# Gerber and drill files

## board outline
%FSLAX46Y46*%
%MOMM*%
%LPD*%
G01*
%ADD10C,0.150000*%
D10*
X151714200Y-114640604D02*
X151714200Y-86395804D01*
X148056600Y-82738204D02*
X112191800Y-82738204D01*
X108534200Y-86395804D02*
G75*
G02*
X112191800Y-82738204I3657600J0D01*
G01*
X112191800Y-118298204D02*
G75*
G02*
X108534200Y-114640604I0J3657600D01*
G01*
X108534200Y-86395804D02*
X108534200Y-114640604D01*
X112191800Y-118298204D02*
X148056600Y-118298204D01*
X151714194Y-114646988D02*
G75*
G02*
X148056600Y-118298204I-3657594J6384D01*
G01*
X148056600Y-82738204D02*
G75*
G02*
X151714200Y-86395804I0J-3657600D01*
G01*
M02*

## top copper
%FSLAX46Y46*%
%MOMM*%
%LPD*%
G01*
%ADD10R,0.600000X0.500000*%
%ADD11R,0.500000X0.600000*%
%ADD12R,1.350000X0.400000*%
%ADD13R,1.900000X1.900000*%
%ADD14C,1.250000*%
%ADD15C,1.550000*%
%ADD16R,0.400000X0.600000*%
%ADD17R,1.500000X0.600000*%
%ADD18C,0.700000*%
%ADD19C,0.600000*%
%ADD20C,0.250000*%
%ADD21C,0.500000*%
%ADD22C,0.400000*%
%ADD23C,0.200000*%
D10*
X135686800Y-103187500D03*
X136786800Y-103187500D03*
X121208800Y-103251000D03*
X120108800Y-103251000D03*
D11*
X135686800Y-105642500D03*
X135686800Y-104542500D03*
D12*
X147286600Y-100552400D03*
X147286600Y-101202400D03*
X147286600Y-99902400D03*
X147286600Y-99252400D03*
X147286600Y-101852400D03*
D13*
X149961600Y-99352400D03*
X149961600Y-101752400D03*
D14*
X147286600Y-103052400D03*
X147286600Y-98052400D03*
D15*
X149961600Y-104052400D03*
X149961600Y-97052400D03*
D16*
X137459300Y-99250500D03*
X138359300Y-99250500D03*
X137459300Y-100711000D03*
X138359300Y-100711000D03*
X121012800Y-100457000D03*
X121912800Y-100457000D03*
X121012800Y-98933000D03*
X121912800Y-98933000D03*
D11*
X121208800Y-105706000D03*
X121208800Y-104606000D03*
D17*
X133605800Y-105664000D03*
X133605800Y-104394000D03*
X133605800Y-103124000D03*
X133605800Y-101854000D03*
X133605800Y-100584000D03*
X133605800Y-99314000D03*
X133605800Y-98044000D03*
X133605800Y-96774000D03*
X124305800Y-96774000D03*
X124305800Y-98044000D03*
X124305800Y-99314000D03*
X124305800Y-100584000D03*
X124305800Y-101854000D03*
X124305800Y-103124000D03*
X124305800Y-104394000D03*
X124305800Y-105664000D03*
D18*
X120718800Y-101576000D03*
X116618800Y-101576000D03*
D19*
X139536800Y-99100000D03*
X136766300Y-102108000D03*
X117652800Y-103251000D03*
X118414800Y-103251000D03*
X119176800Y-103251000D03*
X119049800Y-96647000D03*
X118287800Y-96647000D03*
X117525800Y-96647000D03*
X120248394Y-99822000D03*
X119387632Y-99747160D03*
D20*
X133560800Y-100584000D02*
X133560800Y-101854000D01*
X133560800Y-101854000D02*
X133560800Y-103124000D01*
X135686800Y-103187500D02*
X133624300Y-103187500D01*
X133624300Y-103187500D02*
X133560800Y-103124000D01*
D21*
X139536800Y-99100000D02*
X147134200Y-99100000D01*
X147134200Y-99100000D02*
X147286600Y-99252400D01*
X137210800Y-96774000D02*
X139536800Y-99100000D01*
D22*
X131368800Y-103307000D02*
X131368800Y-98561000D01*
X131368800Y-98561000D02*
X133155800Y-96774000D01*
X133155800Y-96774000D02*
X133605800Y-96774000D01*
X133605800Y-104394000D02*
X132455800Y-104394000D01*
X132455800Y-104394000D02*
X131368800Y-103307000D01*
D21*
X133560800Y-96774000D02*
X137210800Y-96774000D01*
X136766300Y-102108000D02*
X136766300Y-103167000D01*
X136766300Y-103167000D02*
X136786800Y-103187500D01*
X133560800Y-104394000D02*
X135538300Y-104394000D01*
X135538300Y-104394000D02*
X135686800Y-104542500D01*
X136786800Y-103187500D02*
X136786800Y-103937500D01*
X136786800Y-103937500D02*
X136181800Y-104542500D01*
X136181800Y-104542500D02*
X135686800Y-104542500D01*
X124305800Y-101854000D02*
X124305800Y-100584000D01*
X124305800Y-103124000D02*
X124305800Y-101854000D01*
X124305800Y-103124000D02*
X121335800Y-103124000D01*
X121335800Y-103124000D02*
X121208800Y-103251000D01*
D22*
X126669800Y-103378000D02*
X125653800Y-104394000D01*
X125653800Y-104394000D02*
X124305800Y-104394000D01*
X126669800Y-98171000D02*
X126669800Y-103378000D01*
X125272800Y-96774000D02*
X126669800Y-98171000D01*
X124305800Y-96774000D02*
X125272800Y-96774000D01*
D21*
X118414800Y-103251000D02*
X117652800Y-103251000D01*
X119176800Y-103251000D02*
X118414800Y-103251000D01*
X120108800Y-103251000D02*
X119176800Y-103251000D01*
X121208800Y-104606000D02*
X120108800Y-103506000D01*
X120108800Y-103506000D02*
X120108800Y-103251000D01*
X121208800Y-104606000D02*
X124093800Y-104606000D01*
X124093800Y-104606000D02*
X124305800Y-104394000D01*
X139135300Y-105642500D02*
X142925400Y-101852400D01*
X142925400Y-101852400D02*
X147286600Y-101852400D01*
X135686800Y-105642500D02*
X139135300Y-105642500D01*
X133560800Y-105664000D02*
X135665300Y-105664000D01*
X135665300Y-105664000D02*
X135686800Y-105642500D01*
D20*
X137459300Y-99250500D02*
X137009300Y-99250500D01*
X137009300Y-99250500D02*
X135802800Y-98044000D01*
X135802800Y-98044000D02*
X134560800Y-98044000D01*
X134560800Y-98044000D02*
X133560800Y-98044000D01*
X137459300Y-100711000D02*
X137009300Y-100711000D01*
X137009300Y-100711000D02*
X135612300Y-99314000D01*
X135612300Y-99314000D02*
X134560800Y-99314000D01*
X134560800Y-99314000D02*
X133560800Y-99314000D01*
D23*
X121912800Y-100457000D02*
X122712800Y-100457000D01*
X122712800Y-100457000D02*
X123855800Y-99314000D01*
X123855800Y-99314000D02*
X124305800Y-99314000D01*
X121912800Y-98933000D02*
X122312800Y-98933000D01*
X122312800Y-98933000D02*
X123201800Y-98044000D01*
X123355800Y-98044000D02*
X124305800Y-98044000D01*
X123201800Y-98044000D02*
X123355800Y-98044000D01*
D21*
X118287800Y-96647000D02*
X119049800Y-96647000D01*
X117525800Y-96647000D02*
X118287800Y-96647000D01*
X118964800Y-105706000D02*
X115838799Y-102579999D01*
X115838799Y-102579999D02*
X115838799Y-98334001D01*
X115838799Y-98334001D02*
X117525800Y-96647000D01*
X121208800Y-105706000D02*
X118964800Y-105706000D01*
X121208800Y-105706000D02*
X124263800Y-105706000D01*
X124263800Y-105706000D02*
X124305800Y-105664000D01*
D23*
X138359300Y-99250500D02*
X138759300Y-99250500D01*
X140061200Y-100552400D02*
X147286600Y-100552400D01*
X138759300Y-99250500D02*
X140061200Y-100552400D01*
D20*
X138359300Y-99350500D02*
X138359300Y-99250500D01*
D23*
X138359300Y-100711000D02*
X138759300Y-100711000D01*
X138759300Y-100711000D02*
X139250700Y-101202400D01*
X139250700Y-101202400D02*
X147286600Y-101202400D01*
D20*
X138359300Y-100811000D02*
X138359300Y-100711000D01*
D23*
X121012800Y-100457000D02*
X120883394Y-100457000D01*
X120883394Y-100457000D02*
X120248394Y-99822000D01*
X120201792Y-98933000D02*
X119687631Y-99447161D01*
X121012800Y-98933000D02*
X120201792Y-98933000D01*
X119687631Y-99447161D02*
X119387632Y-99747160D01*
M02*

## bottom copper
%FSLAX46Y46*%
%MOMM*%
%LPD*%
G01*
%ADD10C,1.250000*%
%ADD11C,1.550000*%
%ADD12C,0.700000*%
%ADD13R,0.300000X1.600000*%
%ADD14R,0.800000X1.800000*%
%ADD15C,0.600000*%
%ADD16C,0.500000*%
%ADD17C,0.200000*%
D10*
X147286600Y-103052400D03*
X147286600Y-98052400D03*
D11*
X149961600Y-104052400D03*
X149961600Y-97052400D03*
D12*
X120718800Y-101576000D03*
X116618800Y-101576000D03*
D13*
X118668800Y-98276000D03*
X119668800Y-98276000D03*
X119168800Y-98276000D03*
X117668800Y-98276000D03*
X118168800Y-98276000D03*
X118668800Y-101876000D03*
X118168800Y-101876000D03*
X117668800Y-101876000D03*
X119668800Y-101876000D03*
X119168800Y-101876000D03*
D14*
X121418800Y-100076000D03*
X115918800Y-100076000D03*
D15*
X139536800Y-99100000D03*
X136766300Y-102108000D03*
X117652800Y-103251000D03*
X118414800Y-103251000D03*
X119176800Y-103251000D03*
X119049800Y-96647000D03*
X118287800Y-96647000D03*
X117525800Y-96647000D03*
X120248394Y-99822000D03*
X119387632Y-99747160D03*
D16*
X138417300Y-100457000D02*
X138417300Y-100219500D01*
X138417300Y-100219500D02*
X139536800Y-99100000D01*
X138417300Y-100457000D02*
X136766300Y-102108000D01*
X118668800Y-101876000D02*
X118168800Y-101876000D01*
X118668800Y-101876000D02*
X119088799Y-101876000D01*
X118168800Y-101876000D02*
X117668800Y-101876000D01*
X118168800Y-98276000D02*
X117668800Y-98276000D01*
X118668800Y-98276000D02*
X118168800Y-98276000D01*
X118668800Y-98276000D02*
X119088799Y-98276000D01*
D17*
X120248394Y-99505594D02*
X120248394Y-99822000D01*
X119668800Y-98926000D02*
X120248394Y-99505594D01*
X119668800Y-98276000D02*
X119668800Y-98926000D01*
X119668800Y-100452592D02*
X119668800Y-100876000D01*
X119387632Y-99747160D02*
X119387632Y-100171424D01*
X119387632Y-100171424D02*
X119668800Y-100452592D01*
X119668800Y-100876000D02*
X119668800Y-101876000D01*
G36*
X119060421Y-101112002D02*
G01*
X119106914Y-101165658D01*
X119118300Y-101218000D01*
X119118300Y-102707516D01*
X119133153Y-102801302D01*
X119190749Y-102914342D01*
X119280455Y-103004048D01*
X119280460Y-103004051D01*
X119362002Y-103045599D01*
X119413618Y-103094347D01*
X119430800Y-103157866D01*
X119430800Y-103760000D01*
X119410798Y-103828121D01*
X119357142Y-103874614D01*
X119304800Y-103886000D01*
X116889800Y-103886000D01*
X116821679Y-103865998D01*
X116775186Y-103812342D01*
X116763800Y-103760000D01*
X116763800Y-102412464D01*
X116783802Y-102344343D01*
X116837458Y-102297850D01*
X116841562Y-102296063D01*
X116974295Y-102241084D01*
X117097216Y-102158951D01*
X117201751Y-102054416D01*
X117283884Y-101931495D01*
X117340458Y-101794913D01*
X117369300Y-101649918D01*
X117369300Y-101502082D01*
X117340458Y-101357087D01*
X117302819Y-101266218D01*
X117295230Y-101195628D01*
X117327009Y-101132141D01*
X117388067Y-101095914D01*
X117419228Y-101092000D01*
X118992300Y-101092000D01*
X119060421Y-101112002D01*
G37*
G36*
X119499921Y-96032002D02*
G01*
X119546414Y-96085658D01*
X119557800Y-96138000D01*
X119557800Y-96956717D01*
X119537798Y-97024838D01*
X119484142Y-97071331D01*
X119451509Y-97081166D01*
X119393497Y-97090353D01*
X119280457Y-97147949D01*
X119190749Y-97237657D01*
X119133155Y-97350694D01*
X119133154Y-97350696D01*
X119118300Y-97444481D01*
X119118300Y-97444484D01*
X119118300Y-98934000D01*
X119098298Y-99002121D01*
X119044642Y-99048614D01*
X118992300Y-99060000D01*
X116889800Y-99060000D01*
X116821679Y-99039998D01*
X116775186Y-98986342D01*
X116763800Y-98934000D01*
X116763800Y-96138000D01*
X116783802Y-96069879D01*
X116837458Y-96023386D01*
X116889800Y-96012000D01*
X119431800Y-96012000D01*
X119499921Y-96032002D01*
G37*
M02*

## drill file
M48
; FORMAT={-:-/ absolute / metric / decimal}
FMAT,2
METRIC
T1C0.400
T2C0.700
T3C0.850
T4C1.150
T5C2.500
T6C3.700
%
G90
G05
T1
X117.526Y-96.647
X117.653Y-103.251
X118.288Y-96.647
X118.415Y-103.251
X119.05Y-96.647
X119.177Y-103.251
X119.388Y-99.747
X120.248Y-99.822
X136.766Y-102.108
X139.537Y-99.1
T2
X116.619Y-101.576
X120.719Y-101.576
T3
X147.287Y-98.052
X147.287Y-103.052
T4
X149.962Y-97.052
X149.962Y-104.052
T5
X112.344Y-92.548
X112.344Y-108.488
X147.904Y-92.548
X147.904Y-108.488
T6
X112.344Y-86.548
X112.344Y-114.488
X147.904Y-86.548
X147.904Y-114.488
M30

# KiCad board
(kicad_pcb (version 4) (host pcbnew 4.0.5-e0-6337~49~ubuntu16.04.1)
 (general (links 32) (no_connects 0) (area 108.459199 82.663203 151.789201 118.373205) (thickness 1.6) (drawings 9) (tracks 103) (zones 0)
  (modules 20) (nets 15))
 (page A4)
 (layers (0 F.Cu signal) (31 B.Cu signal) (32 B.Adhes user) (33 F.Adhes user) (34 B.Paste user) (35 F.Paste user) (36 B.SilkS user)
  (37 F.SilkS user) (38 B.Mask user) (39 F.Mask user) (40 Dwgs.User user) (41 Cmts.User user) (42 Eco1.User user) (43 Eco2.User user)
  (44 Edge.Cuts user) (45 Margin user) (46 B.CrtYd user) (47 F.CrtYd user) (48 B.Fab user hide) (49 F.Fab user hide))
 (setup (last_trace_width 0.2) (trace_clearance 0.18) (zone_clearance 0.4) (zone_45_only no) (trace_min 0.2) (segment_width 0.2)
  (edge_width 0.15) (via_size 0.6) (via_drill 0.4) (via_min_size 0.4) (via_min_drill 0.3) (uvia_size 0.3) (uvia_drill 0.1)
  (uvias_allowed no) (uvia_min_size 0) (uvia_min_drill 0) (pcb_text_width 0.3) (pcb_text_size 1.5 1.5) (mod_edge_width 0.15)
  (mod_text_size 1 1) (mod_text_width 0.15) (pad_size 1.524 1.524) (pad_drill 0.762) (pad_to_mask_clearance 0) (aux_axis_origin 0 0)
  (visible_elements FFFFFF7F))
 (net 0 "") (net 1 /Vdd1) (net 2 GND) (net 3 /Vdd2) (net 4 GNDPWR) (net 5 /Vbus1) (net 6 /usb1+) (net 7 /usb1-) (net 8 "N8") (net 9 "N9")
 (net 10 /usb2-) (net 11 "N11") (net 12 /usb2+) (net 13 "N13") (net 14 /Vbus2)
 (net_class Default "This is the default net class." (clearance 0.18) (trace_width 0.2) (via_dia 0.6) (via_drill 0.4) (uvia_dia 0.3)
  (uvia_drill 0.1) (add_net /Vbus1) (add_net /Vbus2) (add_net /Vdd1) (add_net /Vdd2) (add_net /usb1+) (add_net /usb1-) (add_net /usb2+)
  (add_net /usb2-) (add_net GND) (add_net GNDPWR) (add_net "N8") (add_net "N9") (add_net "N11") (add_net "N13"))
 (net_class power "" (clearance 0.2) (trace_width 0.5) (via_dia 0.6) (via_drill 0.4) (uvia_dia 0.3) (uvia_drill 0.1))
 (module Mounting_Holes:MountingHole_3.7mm (layer F.Cu) (at 147.9042 86.548204)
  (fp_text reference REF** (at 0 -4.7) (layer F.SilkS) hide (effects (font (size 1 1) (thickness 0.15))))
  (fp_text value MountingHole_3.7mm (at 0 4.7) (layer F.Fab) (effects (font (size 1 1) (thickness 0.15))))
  (pad 1 np_thru_hole circle (at 0 0) (size 3.7 3.7) (drill 3.7) (layers *.Cu *.Mask)))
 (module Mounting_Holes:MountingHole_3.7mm (layer F.Cu) (at 147.9042 114.488204)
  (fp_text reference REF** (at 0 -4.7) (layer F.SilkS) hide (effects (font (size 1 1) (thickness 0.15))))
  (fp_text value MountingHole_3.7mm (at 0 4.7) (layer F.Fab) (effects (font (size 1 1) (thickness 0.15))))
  (pad 1 np_thru_hole circle (at 0 0) (size 3.7 3.7) (drill 3.7) (layers *.Cu *.Mask)))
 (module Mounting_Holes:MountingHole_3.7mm (layer F.Cu) (at 112.3442 114.488204)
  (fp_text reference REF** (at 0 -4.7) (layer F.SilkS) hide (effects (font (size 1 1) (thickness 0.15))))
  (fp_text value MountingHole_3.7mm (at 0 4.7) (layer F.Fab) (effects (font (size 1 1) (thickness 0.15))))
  (pad 1 np_thru_hole circle (at 0 0) (size 3.7 3.7) (drill 3.7) (layers *.Cu *.Mask)))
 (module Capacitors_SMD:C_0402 (layer F.Cu) (at 136.2368 103.1875)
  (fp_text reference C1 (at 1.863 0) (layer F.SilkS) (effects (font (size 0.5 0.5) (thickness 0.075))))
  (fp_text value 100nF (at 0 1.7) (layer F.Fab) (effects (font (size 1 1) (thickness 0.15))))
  (pad 1 smd rect (at -0.55 0) (size 0.6 0.5) (layers F.Cu F.Paste F.Mask) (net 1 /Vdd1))
  (pad 2 smd rect (at 0.55 0) (size 0.6 0.5) (layers F.Cu F.Paste F.Mask) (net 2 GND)))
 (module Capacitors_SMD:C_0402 (layer F.Cu) (at 120.6588 103.251 180)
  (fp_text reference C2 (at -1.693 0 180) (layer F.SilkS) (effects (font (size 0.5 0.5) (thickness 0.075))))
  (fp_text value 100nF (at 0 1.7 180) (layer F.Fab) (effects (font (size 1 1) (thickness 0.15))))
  (pad 1 smd rect (at -0.55 0 180) (size 0.6 0.5) (layers F.Cu F.Paste F.Mask) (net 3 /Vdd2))
  (pad 2 smd rect (at 0.55 0 180) (size 0.6 0.5) (layers F.Cu F.Paste F.Mask) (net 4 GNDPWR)))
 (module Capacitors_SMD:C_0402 (layer F.Cu) (at 135.6868 105.0925 90)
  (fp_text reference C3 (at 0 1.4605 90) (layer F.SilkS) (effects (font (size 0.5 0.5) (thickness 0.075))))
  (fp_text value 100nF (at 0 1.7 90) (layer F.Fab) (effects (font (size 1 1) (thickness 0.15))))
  (pad 1 smd rect (at -0.55 0 90) (size 0.6 0.5) (layers F.Cu F.Paste F.Mask) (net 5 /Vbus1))
  (pad 2 smd rect (at 0.55 0 90) (size 0.6 0.5) (layers F.Cu F.Paste F.Mask) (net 2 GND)))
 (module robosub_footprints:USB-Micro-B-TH (layer F.Cu) (at 146.6116 100.5524 90)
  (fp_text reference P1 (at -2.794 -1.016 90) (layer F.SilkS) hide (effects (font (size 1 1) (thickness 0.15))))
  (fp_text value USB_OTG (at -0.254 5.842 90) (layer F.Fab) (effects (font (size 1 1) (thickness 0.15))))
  (pad 3 smd rect (at 0 0.675 90) (size 0.4 1.35) (layers F.Cu F.Paste F.Mask) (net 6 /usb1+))
  (pad 2 smd rect (at -0.65 0.675 90) (size 0.4 1.35) (layers F.Cu F.Paste F.Mask) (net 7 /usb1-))
  (pad 4 smd rect (at 0.65 0.675 90) (size 0.4 1.35) (layers F.Cu F.Paste F.Mask))
  (pad 5 smd rect (at 1.3 0.675 90) (size 0.4 1.35) (layers F.Cu F.Paste F.Mask) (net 2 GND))
  (pad 1 smd rect (at -1.3 0.675 90) (size 0.4 1.35) (layers F.Cu F.Paste F.Mask) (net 5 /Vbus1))
  (pad "" smd rect (at 1.2 3.35 90) (size 1.9 1.9) (layers F.Cu F.Paste F.Mask))
  (pad "" smd rect (at -1.2 3.35 90) (size 1.9 1.9) (layers F.Cu F.Paste F.Mask))
  (pad "" thru_hole circle (at -2.5 0.675 90) (size 1.25 1.25) (drill 0.85) (layers *.Cu *.Mask F.SilkS))
  (pad "" thru_hole circle (at 2.5 0.675 90) (size 1.25 1.25) (drill 0.85) (layers *.Cu *.Mask F.SilkS))
  (pad "" thru_hole circle (at -3.5 3.35 90) (size 1.55 1.55) (drill 1.15) (layers *.Cu *.Mask F.SilkS))
  (pad "" thru_hole circle (at 3.5 3.35 90) (size 1.55 1.55) (drill 1.15) (layers *.Cu *.Mask F.SilkS)))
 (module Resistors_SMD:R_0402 (layer F.Cu) (at 137.9093 99.2505)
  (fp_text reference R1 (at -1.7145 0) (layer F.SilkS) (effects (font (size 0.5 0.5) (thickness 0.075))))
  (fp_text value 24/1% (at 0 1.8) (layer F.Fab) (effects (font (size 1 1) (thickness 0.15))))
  (pad 1 smd rect (at -0.45 0) (size 0.4 0.6) (layers F.Cu F.Paste F.Mask) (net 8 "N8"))
  (pad 2 smd rect (at 0.45 0) (size 0.4 0.6) (layers F.Cu F.Paste F.Mask) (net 6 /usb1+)))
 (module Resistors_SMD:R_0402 (layer F.Cu) (at 137.9093 100.711)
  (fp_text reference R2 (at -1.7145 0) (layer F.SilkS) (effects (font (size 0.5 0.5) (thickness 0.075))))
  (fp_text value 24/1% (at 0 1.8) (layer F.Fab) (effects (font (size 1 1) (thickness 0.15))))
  (pad 1 smd rect (at -0.45 0) (size 0.4 0.6) (layers F.Cu F.Paste F.Mask) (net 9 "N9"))
  (pad 2 smd rect (at 0.45 0) (size 0.4 0.6) (layers F.Cu F.Paste F.Mask) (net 7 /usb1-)))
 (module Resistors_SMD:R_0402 (layer F.Cu) (at 121.4628 100.457)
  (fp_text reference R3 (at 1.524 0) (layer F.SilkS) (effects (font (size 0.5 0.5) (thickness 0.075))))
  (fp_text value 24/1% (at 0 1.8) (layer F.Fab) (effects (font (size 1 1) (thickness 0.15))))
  (pad 1 smd rect (at -0.45 0) (size 0.4 0.6) (layers F.Cu F.Paste F.Mask) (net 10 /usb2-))
  (pad 2 smd rect (at 0.45 0) (size 0.4 0.6) (layers F.Cu F.Paste F.Mask) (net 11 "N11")))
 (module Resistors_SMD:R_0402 (layer F.Cu) (at 121.4628 98.933)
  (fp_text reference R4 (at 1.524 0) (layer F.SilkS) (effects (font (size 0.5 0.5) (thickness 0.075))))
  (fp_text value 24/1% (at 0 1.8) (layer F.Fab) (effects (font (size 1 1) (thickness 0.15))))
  (pad 1 smd rect (at -0.45 0) (size 0.4 0.6) (layers F.Cu F.Paste F.Mask) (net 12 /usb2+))
  (pad 2 smd rect (at 0.45 0) (size 0.4 0.6) (layers F.Cu F.Paste F.Mask) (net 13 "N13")))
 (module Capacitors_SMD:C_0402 (layer F.Cu) (at 121.2088 105.156 90)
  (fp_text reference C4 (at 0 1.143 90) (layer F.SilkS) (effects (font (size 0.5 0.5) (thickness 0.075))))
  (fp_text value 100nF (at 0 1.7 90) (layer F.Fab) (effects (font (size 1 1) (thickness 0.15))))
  (pad 1 smd rect (at -0.55 0 90) (size 0.6 0.5) (layers F.Cu F.Paste F.Mask) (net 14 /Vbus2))
  (pad 2 smd rect (at 0.55 0 90) (size 0.6 0.5) (layers F.Cu F.Paste F.Mask) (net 4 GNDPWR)))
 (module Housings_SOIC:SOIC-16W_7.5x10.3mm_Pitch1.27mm (layer F.Cu) (at 128.9558 101.219 180)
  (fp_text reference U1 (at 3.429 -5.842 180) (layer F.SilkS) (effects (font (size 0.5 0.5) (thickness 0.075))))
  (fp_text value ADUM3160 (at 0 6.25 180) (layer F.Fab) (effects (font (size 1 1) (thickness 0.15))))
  (pad 1 smd rect (at -4.65 -4.445 180) (size 1.5 0.6) (layers F.Cu F.Paste F.Mask) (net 5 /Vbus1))
  (pad 2 smd rect (at -4.65 -3.175 180) (size 1.5 0.6) (layers F.Cu F.Paste F.Mask) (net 2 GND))
  (pad 3 smd rect (at -4.65 -1.905 180) (size 1.5 0.6) (layers F.Cu F.Paste F.Mask) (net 1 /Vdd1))
  (pad 4 smd rect (at -4.65 -0.635 180) (size 1.5 0.6) (layers F.Cu F.Paste F.Mask) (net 1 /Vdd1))
  (pad 5 smd rect (at -4.65 0.635 180) (size 1.5 0.6) (layers F.Cu F.Paste F.Mask) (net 1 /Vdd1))
  (pad 6 smd rect (at -4.65 1.905 180) (size 1.5 0.6) (layers F.Cu F.Paste F.Mask) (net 9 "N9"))
  (pad 7 smd rect (at -4.65 3.175 180) (size 1.5 0.6) (layers F.Cu F.Paste F.Mask) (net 8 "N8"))
  (pad 8 smd rect (at -4.65 4.445 180) (size 1.5 0.6) (layers F.Cu F.Paste F.Mask) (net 2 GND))
  (pad 9 smd rect (at 4.65 4.445 180) (size 1.5 0.6) (layers F.Cu F.Paste F.Mask) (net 4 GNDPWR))
  (pad 10 smd rect (at 4.65 3.175 180) (size 1.5 0.6) (layers F.Cu F.Paste F.Mask) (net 13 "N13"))
  (pad 11 smd rect (at 4.65 1.905 180) (size 1.5 0.6) (layers F.Cu F.Paste F.Mask) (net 11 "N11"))
  (pad 12 smd rect (at 4.65 0.635 180) (size 1.5 0.6) (layers F.Cu F.Paste F.Mask) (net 3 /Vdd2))
  (pad 13 smd rect (at 4.65 -0.635 180) (size 1.5 0.6) (layers F.Cu F.Paste F.Mask) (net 3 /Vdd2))
  (pad 14 smd rect (at 4.65 -1.905 180) (size 1.5 0.6) (layers F.Cu F.Paste F.Mask) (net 3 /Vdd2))
  (pad 15 smd rect (at 4.65 -3.175 180) (size 1.5 0.6) (layers F.Cu F.Paste F.Mask) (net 4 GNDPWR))
  (pad 16 smd rect (at 4.65 -4.445 180) (size 1.5 0.6) (layers F.Cu F.Paste F.Mask) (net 14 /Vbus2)))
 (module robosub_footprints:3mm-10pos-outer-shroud (layer B.Cu) (at 118.6688 100.076)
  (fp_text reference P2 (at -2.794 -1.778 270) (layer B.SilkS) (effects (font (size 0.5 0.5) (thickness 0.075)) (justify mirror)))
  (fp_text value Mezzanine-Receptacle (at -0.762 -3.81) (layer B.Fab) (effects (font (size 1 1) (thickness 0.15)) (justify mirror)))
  (pad "" thru_hole circle (at 2.05 1.5) (size 0.7 0.7) (drill 0.7) (layers *.Cu *.Mask))
  (pad "" thru_hole circle (at -2.05 1.5) (size 0.7 0.7) (drill 0.7) (layers *.Cu *.Mask))
  (pad 5 smd rect (at 0 -1.8) (size 0.3 1.6) (layers B.Cu B.Paste B.Mask) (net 14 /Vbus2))
  (pad 9 smd rect (at 1 -1.8) (size 0.3 1.6) (layers B.Cu B.Paste B.Mask) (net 10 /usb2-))
  (pad 7 smd rect (at 0.5 -1.8) (size 0.3 1.6) (layers B.Cu B.Paste B.Mask) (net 14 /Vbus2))
  (pad 1 smd rect (at -1 -1.8) (size 0.3 1.6) (layers B.Cu B.Paste B.Mask) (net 14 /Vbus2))
  (pad 3 smd rect (at -0.5 -1.8) (size 0.3 1.6) (layers B.Cu B.Paste B.Mask) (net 14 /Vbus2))
  (pad 6 smd rect (at 0 1.8) (size 0.3 1.6) (layers B.Cu B.Paste B.Mask) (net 4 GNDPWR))
  (pad 4 smd rect (at -0.5 1.8) (size 0.3 1.6) (layers B.Cu B.Paste B.Mask) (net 4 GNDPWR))
  (pad 2 smd rect (at -1 1.8) (size 0.3 1.6) (layers B.Cu B.Paste B.Mask) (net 4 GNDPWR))
  (pad 10 smd rect (at 1 1.8) (size 0.3 1.6) (layers B.Cu B.Paste B.Mask) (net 12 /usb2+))
  (pad 8 smd rect (at 0.5 1.8) (size 0.3 1.6) (layers B.Cu B.Paste B.Mask) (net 4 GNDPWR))
  (pad "" smd rect (at 2.75 0) (size 0.8 1.8) (layers B.Cu B.Paste B.Mask))
  (pad "" smd rect (at -2.75 0) (size 0.8 1.8) (layers B.Cu B.Paste B.Mask)))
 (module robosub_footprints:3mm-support (layer B.Cu) (at 147.9042 108.488204)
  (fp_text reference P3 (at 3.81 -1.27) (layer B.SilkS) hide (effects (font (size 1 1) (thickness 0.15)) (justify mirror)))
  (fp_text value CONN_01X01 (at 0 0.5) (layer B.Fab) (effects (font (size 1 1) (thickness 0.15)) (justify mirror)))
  (pad "" np_thru_hole circle (at 0 0) (size 2.5 2.5) (drill 2.5) (layers *.Cu *.Mask)))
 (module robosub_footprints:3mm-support (layer B.Cu) (at 147.9042 92.548204)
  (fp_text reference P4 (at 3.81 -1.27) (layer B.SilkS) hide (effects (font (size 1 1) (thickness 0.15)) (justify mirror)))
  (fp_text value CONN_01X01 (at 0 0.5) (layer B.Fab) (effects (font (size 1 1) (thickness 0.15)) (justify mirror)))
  (pad "" np_thru_hole circle (at 0 0) (size 2.5 2.5) (drill 2.5) (layers *.Cu *.Mask)))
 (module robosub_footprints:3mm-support (layer B.Cu) (at 112.3442 108.488204)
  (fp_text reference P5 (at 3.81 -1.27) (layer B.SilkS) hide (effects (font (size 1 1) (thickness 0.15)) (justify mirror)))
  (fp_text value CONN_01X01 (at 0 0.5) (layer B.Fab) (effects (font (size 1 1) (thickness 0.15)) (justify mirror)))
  (pad "" np_thru_hole circle (at 0 0) (size 2.5 2.5) (drill 2.5) (layers *.Cu *.Mask)))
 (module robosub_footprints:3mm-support (layer B.Cu) (at 112.3442 92.548204)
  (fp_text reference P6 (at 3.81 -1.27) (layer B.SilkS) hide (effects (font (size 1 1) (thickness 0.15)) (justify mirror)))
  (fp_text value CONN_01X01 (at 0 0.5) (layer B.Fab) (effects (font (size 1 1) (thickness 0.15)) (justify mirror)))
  (pad "" np_thru_hole circle (at 0 0) (size 2.5 2.5) (drill 2.5) (layers *.Cu *.Mask)))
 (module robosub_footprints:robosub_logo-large (layer F.Cu) (at 125.476 112.5982)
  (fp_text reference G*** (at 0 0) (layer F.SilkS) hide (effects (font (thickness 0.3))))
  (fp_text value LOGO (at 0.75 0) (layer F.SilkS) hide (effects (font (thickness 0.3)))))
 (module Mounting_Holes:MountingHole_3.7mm (layer F.Cu) (at 112.3442 86.548204)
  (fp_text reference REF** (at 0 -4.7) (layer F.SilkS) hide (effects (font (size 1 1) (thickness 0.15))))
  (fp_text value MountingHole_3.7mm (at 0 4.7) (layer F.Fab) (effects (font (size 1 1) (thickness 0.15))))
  (pad 1 np_thru_hole circle (at 0 0) (size 3.7 3.7) (drill 3.7) (layers *.Cu *.Mask)))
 (gr_line (start 151.7142 114.640604) (end 151.7142 86.395804) (layer Edge.Cuts) (width 0.15))
 (gr_line (start 148.0566 82.738204) (end 112.1918 82.738204) (layer Edge.Cuts) (width 0.15))
 (gr_arc (start 112.1918 86.395804) (end 112.1918 82.738204) (angle -90) (layer Edge.Cuts) (width 0.15))
 (gr_arc (start 112.1918 114.640604) (end 108.5342 114.640604) (angle -90) (layer Edge.Cuts) (width 0.15))
 (gr_line (start 108.5342 86.395804) (end 108.5342 114.640604) (layer Edge.Cuts) (width 0.15))
 (gr_line (start 112.1918 118.298204) (end 148.0566 118.298204) (layer Edge.Cuts) (width 0.15))
 (gr_arc (start 148.0566 114.640604) (end 148.0566 118.298204) (angle -89.9) (layer Edge.Cuts) (width 0.15))
 (gr_arc (start 148.0566 86.395804) (end 151.7142 86.395804) (angle -90) (layer Edge.Cuts) (width 0.15))
 (segment (start 133.5608 100.584) (end 133.5608 101.854) (width 0.25) (layer F.Cu) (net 1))
 (segment (start 133.5608 101.854) (end 133.5608 103.124) (width 0.25) (layer F.Cu) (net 1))
 (segment (start 135.6868 103.1875) (end 133.6243 103.1875) (width 0.25) (layer F.Cu) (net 1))
 (segment (start 133.6243 103.1875) (end 133.5608 103.124) (width 0.25) (layer F.Cu) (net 1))
 (segment (start 139.5368 99.1) (end 147.1342 99.1) (width 0.5) (layer F.Cu) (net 2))
 (segment (start 147.1342 99.1) (end 147.2866 99.2524) (width 0.5) (layer F.Cu) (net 2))
 (segment (start 138.4173 100.457) (end 138.4173 100.2195) (width 0.5) (layer B.Cu) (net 2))
 (segment (start 138.4173 100.2195) (end 139.5368 99.1) (width 0.5) (layer B.Cu) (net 2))
 (via (at 139.5368 99.1) (size 0.6) (drill 0.4) (layers F.Cu B.Cu) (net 2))
 (segment (start 137.2108 96.774) (end 139.5368 99.1) (width 0.5) (layer F.Cu) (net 2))
 (segment (start 131.3688 103.307) (end 131.3688 98.561) (width 0.4) (layer F.Cu) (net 2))
 (segment (start 131.3688 98.561) (end 133.1558 96.774) (width 0.4) (layer F.Cu) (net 2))
 (segment (start 133.1558 96.774) (end 133.6058 96.774) (width 0.4) (layer F.Cu) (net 2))
 (segment (start 133.6058 104.394) (end 132.4558 104.394) (width 0.4) (layer F.Cu) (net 2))
 (segment (start 132.4558 104.394) (end 131.3688 103.307) (width 0.4) (layer F.Cu) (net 2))
 (segment (start 133.5608 96.774) (end 137.2108 96.774) (width 0.5) (layer F.Cu) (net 2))
 (segment (start 136.7663 102.108) (end 136.7663 103.167) (width 0.5) (layer F.Cu) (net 2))
 (segment (start 136.7663 103.167) (end 136.7868 103.1875) (width 0.5) (layer F.Cu) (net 2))
 (segment (start 138.4173 100.457) (end 136.7663 102.108) (width 0.5) (layer B.Cu) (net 2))
 (via (at 136.7663 102.108) (size 0.6) (drill 0.4) (layers F.Cu B.Cu) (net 2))
 (segment (start 133.5608 104.394) (end 135.5383 104.394) (width 0.5) (layer F.Cu) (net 2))
 (segment (start 135.5383 104.394) (end 135.6868 104.5425) (width 0.5) (layer F.Cu) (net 2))
 (segment (start 136.7868 103.1875) (end 136.7868 103.9375) (width 0.5) (layer F.Cu) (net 2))
 (segment (start 136.7868 103.9375) (end 136.1818 104.5425) (width 0.5) (layer F.Cu) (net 2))
 (segment (start 136.1818 104.5425) (end 135.6868 104.5425) (width 0.5) (layer F.Cu) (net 2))
 (segment (start 124.3058 101.854) (end 124.3058 100.584) (width 0.5) (layer F.Cu) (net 3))
 (segment (start 124.3058 103.124) (end 124.3058 101.854) (width 0.5) (layer F.Cu) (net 3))
 (segment (start 124.3058 103.124) (end 121.3358 103.124) (width 0.5) (layer F.Cu) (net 3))
 (segment (start 121.3358 103.124) (end 121.2088 103.251) (width 0.5) (layer F.Cu) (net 3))
 (segment (start 126.6698 103.378) (end 125.6538 104.394) (width 0.4) (layer F.Cu) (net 4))
 (segment (start 125.6538 104.394) (end 124.3058 104.394) (width 0.4) (layer F.Cu) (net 4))
 (segment (start 126.6698 98.171) (end 126.6698 103.378) (width 0.4) (layer F.Cu) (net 4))
 (segment (start 125.2728 96.774) (end 126.6698 98.171) (width 0.4) (layer F.Cu) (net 4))
 (segment (start 124.3058 96.774) (end 125.2728 96.774) (width 0.4) (layer F.Cu) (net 4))
 (segment (start 118.6688 101.876) (end 118.1688 101.876) (width 0.5) (layer B.Cu) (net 4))
 (segment (start 118.4148 103.251) (end 117.6528 103.251) (width 0.5) (layer F.Cu) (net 4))
 (via (at 117.6528 103.251) (size 0.6) (drill 0.4) (layers F.Cu B.Cu) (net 4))
 (segment (start 119.1768 103.251) (end 118.4148 103.251) (width 0.5) (layer F.Cu) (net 4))
 (via (at 118.4148 103.251) (size 0.6) (drill 0.4) (layers F.Cu B.Cu) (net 4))
 (segment (start 120.1088 103.251) (end 119.1768 103.251) (width 0.5) (layer F.Cu) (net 4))
 (via (at 119.1768 103.251) (size 0.6) (drill 0.4) (layers F.Cu B.Cu) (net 4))
 (segment (start 118.6688 101.876) (end 119.088799 101.876) (width 0.5) (layer B.Cu) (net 4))
 (segment (start 118.1688 101.876) (end 117.6688 101.876) (width 0.5) (layer B.Cu) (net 4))
 (segment (start 121.2088 104.606) (end 120.1088 103.506) (width 0.5) (layer F.Cu) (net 4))
 (segment (start 120.1088 103.506) (end 120.1088 103.251) (width 0.5) (layer F.Cu) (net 4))
 (segment (start 121.2088 104.606) (end 124.0938 104.606) (width 0.5) (layer F.Cu) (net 4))
 (segment (start 124.0938 104.606) (end 124.3058 104.394) (width 0.5) (layer F.Cu) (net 4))
 (segment (start 139.1353 105.6425) (end 142.9254 101.8524) (width 0.5) (layer F.Cu) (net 5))
 (segment (start 142.9254 101.8524) (end 147.2866 101.8524) (width 0.5) (layer F.Cu) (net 5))
 (segment (start 135.6868 105.6425) (end 139.1353 105.6425) (width 0.5) (layer F.Cu) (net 5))
 (segment (start 133.5608 105.664) (end 135.6653 105.664) (width 0.5) (layer F.Cu) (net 5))
 (segment (start 135.6653 105.664) (end 135.6868 105.6425) (width 0.5) (layer F.Cu) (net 5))
 (segment (start 137.4593 99.2505) (end 137.0093 99.2505) (width 0.25) (layer F.Cu) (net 8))
 (segment (start 137.0093 99.2505) (end 135.8028 98.044) (width 0.25) (layer F.Cu) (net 8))
 (segment (start 135.8028 98.044) (end 134.5608 98.044) (width 0.25) (layer F.Cu) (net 8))
 (segment (start 134.5608 98.044) (end 133.5608 98.044) (width 0.25) (layer F.Cu) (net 8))
 (segment (start 137.4593 100.711) (end 137.0093 100.711) (width 0.25) (layer F.Cu) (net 9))
 (segment (start 137.0093 100.711) (end 135.6123 99.314) (width 0.25) (layer F.Cu) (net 9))
 (segment (start 135.6123 99.314) (end 134.5608 99.314) (width 0.25) (layer F.Cu) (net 9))
 (segment (start 134.5608 99.314) (end 133.5608 99.314) (width 0.25) (layer F.Cu) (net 9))
 (segment (start 121.9128 100.457) (end 122.7128 100.457) (width 0.2) (layer F.Cu) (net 11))
 (segment (start 122.7128 100.457) (end 123.8558 99.314) (width 0.2) (layer F.Cu) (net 11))
 (segment (start 123.8558 99.314) (end 124.3058 99.314) (width 0.2) (layer F.Cu) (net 11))
 (segment (start 121.9128 98.933) (end 122.3128 98.933) (width 0.2) (layer F.Cu) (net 13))
 (segment (start 122.3128 98.933) (end 123.2018 98.044) (width 0.2) (layer F.Cu) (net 13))
 (segment (start 123.3558 98.044) (end 124.3058 98.044) (width 0.2) (layer F.Cu) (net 13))
 (segment (start 123.2018 98.044) (end 123.3558 98.044) (width 0.2) (layer F.Cu) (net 13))
 (segment (start 118.1688 98.276) (end 117.6688 98.276) (width 0.5) (layer B.Cu) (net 14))
 (segment (start 118.6688 98.276) (end 118.1688 98.276) (width 0.5) (layer B.Cu) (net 14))
 (segment (start 118.6688 98.276) (end 119.088799 98.276) (width 0.5) (layer B.Cu) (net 14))
 (segment (start 118.2878 96.647) (end 119.0498 96.647) (width 0.5) (layer F.Cu) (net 14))
 (via (at 119.0498 96.647) (size 0.6) (drill 0.4) (layers F.Cu B.Cu) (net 14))
 (segment (start 117.5258 96.647) (end 118.2878 96.647) (width 0.5) (layer F.Cu) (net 14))
 (via (at 118.2878 96.647) (size 0.6) (drill 0.4) (layers F.Cu B.Cu) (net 14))
 (segment (start 118.9648 105.706) (end 115.838799 102.579999) (width 0.5) (layer F.Cu) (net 14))
 (segment (start 115.838799 102.579999) (end 115.838799 98.334001) (width 0.5) (layer F.Cu) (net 14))
 (segment (start 115.838799 98.334001) (end 117.5258 96.647) (width 0.5) (layer F.Cu) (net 14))
 (via (at 117.5258 96.647) (size 0.6) (drill 0.4) (layers F.Cu B.Cu) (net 14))
 (segment (start 121.2088 105.706) (end 118.9648 105.706) (width 0.5) (layer F.Cu) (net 14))
 (segment (start 121.2088 105.706) (end 124.2638 105.706) (width 0.5) (layer F.Cu) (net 14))
 (segment (start 124.2638 105.706) (end 124.3058 105.664) (width 0.5) (layer F.Cu) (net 14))
 (segment (start 138.3593 99.2505) (end 138.7593 99.2505) (width 0.2) (layer F.Cu) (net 6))
 (segment (start 140.0612 100.5524) (end 147.2866 100.5524) (width 0.2) (layer F.Cu) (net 6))
 (segment (start 138.7593 99.2505) (end 140.0612 100.5524) (width 0.2) (layer F.Cu) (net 6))
 (segment (start 138.3593 99.3505) (end 138.3593 99.2505) (width 0.25) (layer F.Cu) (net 6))
 (segment (start 138.3593 100.711) (end 138.7593 100.711) (width 0.2) (layer F.Cu) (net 7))
 (segment (start 138.7593 100.711) (end 139.2507 101.2024) (width 0.2) (layer F.Cu) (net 7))
 (segment (start 139.2507 101.2024) (end 147.2866 101.2024) (width 0.2) (layer F.Cu) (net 7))
 (segment (start 138.3593 100.811) (end 138.3593 100.711) (width 0.25) (layer F.Cu) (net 7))
 (segment (start 120.248394 99.505594) (end 120.248394 99.822) (width 0.2) (layer B.Cu) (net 10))
 (segment (start 121.0128 100.457) (end 120.883394 100.457) (width 0.2) (layer F.Cu) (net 10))
 (segment (start 120.883394 100.457) (end 120.248394 99.822) (width 0.2) (layer F.Cu) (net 10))
 (via (at 120.248394 99.822) (size 0.6) (drill 0.4) (layers F.Cu B.Cu) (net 10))
 (segment (start 119.6688 98.926) (end 120.248394 99.505594) (width 0.2) (layer B.Cu) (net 10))
 (segment (start 119.6688 98.276) (end 119.6688 98.926) (width 0.2) (layer B.Cu) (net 10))
 (segment (start 119.6688 100.452592) (end 119.6688 100.876) (width 0.2) (layer B.Cu) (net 12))
 (segment (start 119.387632 99.74716) (end 119.387632 100.171424) (width 0.2) (layer B.Cu) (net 12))
 (segment (start 119.387632 100.171424) (end 119.6688 100.452592) (width 0.2) (layer B.Cu) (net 12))
 (segment (start 119.6688 100.876) (end 119.6688 101.876) (width 0.2) (layer B.Cu) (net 12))
 (segment (start 120.201792 98.933) (end 119.687631 99.447161) (width 0.2) (layer F.Cu) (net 12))
 (segment (start 121.0128 98.933) (end 120.201792 98.933) (width 0.2) (layer F.Cu) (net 12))
 (via (at 119.387632 99.74716) (size 0.6) (drill 0.4) (layers F.Cu B.Cu) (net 12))
 (segment (start 119.687631 99.447161) (end 119.387632 99.74716) (width 0.2) (layer F.Cu) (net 12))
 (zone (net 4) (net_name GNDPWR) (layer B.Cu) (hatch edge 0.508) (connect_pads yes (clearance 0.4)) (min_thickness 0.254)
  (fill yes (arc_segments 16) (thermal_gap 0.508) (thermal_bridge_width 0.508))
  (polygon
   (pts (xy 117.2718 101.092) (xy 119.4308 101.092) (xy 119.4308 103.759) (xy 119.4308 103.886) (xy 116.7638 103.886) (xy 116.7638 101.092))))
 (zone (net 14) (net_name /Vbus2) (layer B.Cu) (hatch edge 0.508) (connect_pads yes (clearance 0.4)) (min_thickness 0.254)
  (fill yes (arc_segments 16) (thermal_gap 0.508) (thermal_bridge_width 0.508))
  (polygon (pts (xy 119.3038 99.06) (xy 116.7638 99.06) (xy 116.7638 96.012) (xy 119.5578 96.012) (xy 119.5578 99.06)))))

